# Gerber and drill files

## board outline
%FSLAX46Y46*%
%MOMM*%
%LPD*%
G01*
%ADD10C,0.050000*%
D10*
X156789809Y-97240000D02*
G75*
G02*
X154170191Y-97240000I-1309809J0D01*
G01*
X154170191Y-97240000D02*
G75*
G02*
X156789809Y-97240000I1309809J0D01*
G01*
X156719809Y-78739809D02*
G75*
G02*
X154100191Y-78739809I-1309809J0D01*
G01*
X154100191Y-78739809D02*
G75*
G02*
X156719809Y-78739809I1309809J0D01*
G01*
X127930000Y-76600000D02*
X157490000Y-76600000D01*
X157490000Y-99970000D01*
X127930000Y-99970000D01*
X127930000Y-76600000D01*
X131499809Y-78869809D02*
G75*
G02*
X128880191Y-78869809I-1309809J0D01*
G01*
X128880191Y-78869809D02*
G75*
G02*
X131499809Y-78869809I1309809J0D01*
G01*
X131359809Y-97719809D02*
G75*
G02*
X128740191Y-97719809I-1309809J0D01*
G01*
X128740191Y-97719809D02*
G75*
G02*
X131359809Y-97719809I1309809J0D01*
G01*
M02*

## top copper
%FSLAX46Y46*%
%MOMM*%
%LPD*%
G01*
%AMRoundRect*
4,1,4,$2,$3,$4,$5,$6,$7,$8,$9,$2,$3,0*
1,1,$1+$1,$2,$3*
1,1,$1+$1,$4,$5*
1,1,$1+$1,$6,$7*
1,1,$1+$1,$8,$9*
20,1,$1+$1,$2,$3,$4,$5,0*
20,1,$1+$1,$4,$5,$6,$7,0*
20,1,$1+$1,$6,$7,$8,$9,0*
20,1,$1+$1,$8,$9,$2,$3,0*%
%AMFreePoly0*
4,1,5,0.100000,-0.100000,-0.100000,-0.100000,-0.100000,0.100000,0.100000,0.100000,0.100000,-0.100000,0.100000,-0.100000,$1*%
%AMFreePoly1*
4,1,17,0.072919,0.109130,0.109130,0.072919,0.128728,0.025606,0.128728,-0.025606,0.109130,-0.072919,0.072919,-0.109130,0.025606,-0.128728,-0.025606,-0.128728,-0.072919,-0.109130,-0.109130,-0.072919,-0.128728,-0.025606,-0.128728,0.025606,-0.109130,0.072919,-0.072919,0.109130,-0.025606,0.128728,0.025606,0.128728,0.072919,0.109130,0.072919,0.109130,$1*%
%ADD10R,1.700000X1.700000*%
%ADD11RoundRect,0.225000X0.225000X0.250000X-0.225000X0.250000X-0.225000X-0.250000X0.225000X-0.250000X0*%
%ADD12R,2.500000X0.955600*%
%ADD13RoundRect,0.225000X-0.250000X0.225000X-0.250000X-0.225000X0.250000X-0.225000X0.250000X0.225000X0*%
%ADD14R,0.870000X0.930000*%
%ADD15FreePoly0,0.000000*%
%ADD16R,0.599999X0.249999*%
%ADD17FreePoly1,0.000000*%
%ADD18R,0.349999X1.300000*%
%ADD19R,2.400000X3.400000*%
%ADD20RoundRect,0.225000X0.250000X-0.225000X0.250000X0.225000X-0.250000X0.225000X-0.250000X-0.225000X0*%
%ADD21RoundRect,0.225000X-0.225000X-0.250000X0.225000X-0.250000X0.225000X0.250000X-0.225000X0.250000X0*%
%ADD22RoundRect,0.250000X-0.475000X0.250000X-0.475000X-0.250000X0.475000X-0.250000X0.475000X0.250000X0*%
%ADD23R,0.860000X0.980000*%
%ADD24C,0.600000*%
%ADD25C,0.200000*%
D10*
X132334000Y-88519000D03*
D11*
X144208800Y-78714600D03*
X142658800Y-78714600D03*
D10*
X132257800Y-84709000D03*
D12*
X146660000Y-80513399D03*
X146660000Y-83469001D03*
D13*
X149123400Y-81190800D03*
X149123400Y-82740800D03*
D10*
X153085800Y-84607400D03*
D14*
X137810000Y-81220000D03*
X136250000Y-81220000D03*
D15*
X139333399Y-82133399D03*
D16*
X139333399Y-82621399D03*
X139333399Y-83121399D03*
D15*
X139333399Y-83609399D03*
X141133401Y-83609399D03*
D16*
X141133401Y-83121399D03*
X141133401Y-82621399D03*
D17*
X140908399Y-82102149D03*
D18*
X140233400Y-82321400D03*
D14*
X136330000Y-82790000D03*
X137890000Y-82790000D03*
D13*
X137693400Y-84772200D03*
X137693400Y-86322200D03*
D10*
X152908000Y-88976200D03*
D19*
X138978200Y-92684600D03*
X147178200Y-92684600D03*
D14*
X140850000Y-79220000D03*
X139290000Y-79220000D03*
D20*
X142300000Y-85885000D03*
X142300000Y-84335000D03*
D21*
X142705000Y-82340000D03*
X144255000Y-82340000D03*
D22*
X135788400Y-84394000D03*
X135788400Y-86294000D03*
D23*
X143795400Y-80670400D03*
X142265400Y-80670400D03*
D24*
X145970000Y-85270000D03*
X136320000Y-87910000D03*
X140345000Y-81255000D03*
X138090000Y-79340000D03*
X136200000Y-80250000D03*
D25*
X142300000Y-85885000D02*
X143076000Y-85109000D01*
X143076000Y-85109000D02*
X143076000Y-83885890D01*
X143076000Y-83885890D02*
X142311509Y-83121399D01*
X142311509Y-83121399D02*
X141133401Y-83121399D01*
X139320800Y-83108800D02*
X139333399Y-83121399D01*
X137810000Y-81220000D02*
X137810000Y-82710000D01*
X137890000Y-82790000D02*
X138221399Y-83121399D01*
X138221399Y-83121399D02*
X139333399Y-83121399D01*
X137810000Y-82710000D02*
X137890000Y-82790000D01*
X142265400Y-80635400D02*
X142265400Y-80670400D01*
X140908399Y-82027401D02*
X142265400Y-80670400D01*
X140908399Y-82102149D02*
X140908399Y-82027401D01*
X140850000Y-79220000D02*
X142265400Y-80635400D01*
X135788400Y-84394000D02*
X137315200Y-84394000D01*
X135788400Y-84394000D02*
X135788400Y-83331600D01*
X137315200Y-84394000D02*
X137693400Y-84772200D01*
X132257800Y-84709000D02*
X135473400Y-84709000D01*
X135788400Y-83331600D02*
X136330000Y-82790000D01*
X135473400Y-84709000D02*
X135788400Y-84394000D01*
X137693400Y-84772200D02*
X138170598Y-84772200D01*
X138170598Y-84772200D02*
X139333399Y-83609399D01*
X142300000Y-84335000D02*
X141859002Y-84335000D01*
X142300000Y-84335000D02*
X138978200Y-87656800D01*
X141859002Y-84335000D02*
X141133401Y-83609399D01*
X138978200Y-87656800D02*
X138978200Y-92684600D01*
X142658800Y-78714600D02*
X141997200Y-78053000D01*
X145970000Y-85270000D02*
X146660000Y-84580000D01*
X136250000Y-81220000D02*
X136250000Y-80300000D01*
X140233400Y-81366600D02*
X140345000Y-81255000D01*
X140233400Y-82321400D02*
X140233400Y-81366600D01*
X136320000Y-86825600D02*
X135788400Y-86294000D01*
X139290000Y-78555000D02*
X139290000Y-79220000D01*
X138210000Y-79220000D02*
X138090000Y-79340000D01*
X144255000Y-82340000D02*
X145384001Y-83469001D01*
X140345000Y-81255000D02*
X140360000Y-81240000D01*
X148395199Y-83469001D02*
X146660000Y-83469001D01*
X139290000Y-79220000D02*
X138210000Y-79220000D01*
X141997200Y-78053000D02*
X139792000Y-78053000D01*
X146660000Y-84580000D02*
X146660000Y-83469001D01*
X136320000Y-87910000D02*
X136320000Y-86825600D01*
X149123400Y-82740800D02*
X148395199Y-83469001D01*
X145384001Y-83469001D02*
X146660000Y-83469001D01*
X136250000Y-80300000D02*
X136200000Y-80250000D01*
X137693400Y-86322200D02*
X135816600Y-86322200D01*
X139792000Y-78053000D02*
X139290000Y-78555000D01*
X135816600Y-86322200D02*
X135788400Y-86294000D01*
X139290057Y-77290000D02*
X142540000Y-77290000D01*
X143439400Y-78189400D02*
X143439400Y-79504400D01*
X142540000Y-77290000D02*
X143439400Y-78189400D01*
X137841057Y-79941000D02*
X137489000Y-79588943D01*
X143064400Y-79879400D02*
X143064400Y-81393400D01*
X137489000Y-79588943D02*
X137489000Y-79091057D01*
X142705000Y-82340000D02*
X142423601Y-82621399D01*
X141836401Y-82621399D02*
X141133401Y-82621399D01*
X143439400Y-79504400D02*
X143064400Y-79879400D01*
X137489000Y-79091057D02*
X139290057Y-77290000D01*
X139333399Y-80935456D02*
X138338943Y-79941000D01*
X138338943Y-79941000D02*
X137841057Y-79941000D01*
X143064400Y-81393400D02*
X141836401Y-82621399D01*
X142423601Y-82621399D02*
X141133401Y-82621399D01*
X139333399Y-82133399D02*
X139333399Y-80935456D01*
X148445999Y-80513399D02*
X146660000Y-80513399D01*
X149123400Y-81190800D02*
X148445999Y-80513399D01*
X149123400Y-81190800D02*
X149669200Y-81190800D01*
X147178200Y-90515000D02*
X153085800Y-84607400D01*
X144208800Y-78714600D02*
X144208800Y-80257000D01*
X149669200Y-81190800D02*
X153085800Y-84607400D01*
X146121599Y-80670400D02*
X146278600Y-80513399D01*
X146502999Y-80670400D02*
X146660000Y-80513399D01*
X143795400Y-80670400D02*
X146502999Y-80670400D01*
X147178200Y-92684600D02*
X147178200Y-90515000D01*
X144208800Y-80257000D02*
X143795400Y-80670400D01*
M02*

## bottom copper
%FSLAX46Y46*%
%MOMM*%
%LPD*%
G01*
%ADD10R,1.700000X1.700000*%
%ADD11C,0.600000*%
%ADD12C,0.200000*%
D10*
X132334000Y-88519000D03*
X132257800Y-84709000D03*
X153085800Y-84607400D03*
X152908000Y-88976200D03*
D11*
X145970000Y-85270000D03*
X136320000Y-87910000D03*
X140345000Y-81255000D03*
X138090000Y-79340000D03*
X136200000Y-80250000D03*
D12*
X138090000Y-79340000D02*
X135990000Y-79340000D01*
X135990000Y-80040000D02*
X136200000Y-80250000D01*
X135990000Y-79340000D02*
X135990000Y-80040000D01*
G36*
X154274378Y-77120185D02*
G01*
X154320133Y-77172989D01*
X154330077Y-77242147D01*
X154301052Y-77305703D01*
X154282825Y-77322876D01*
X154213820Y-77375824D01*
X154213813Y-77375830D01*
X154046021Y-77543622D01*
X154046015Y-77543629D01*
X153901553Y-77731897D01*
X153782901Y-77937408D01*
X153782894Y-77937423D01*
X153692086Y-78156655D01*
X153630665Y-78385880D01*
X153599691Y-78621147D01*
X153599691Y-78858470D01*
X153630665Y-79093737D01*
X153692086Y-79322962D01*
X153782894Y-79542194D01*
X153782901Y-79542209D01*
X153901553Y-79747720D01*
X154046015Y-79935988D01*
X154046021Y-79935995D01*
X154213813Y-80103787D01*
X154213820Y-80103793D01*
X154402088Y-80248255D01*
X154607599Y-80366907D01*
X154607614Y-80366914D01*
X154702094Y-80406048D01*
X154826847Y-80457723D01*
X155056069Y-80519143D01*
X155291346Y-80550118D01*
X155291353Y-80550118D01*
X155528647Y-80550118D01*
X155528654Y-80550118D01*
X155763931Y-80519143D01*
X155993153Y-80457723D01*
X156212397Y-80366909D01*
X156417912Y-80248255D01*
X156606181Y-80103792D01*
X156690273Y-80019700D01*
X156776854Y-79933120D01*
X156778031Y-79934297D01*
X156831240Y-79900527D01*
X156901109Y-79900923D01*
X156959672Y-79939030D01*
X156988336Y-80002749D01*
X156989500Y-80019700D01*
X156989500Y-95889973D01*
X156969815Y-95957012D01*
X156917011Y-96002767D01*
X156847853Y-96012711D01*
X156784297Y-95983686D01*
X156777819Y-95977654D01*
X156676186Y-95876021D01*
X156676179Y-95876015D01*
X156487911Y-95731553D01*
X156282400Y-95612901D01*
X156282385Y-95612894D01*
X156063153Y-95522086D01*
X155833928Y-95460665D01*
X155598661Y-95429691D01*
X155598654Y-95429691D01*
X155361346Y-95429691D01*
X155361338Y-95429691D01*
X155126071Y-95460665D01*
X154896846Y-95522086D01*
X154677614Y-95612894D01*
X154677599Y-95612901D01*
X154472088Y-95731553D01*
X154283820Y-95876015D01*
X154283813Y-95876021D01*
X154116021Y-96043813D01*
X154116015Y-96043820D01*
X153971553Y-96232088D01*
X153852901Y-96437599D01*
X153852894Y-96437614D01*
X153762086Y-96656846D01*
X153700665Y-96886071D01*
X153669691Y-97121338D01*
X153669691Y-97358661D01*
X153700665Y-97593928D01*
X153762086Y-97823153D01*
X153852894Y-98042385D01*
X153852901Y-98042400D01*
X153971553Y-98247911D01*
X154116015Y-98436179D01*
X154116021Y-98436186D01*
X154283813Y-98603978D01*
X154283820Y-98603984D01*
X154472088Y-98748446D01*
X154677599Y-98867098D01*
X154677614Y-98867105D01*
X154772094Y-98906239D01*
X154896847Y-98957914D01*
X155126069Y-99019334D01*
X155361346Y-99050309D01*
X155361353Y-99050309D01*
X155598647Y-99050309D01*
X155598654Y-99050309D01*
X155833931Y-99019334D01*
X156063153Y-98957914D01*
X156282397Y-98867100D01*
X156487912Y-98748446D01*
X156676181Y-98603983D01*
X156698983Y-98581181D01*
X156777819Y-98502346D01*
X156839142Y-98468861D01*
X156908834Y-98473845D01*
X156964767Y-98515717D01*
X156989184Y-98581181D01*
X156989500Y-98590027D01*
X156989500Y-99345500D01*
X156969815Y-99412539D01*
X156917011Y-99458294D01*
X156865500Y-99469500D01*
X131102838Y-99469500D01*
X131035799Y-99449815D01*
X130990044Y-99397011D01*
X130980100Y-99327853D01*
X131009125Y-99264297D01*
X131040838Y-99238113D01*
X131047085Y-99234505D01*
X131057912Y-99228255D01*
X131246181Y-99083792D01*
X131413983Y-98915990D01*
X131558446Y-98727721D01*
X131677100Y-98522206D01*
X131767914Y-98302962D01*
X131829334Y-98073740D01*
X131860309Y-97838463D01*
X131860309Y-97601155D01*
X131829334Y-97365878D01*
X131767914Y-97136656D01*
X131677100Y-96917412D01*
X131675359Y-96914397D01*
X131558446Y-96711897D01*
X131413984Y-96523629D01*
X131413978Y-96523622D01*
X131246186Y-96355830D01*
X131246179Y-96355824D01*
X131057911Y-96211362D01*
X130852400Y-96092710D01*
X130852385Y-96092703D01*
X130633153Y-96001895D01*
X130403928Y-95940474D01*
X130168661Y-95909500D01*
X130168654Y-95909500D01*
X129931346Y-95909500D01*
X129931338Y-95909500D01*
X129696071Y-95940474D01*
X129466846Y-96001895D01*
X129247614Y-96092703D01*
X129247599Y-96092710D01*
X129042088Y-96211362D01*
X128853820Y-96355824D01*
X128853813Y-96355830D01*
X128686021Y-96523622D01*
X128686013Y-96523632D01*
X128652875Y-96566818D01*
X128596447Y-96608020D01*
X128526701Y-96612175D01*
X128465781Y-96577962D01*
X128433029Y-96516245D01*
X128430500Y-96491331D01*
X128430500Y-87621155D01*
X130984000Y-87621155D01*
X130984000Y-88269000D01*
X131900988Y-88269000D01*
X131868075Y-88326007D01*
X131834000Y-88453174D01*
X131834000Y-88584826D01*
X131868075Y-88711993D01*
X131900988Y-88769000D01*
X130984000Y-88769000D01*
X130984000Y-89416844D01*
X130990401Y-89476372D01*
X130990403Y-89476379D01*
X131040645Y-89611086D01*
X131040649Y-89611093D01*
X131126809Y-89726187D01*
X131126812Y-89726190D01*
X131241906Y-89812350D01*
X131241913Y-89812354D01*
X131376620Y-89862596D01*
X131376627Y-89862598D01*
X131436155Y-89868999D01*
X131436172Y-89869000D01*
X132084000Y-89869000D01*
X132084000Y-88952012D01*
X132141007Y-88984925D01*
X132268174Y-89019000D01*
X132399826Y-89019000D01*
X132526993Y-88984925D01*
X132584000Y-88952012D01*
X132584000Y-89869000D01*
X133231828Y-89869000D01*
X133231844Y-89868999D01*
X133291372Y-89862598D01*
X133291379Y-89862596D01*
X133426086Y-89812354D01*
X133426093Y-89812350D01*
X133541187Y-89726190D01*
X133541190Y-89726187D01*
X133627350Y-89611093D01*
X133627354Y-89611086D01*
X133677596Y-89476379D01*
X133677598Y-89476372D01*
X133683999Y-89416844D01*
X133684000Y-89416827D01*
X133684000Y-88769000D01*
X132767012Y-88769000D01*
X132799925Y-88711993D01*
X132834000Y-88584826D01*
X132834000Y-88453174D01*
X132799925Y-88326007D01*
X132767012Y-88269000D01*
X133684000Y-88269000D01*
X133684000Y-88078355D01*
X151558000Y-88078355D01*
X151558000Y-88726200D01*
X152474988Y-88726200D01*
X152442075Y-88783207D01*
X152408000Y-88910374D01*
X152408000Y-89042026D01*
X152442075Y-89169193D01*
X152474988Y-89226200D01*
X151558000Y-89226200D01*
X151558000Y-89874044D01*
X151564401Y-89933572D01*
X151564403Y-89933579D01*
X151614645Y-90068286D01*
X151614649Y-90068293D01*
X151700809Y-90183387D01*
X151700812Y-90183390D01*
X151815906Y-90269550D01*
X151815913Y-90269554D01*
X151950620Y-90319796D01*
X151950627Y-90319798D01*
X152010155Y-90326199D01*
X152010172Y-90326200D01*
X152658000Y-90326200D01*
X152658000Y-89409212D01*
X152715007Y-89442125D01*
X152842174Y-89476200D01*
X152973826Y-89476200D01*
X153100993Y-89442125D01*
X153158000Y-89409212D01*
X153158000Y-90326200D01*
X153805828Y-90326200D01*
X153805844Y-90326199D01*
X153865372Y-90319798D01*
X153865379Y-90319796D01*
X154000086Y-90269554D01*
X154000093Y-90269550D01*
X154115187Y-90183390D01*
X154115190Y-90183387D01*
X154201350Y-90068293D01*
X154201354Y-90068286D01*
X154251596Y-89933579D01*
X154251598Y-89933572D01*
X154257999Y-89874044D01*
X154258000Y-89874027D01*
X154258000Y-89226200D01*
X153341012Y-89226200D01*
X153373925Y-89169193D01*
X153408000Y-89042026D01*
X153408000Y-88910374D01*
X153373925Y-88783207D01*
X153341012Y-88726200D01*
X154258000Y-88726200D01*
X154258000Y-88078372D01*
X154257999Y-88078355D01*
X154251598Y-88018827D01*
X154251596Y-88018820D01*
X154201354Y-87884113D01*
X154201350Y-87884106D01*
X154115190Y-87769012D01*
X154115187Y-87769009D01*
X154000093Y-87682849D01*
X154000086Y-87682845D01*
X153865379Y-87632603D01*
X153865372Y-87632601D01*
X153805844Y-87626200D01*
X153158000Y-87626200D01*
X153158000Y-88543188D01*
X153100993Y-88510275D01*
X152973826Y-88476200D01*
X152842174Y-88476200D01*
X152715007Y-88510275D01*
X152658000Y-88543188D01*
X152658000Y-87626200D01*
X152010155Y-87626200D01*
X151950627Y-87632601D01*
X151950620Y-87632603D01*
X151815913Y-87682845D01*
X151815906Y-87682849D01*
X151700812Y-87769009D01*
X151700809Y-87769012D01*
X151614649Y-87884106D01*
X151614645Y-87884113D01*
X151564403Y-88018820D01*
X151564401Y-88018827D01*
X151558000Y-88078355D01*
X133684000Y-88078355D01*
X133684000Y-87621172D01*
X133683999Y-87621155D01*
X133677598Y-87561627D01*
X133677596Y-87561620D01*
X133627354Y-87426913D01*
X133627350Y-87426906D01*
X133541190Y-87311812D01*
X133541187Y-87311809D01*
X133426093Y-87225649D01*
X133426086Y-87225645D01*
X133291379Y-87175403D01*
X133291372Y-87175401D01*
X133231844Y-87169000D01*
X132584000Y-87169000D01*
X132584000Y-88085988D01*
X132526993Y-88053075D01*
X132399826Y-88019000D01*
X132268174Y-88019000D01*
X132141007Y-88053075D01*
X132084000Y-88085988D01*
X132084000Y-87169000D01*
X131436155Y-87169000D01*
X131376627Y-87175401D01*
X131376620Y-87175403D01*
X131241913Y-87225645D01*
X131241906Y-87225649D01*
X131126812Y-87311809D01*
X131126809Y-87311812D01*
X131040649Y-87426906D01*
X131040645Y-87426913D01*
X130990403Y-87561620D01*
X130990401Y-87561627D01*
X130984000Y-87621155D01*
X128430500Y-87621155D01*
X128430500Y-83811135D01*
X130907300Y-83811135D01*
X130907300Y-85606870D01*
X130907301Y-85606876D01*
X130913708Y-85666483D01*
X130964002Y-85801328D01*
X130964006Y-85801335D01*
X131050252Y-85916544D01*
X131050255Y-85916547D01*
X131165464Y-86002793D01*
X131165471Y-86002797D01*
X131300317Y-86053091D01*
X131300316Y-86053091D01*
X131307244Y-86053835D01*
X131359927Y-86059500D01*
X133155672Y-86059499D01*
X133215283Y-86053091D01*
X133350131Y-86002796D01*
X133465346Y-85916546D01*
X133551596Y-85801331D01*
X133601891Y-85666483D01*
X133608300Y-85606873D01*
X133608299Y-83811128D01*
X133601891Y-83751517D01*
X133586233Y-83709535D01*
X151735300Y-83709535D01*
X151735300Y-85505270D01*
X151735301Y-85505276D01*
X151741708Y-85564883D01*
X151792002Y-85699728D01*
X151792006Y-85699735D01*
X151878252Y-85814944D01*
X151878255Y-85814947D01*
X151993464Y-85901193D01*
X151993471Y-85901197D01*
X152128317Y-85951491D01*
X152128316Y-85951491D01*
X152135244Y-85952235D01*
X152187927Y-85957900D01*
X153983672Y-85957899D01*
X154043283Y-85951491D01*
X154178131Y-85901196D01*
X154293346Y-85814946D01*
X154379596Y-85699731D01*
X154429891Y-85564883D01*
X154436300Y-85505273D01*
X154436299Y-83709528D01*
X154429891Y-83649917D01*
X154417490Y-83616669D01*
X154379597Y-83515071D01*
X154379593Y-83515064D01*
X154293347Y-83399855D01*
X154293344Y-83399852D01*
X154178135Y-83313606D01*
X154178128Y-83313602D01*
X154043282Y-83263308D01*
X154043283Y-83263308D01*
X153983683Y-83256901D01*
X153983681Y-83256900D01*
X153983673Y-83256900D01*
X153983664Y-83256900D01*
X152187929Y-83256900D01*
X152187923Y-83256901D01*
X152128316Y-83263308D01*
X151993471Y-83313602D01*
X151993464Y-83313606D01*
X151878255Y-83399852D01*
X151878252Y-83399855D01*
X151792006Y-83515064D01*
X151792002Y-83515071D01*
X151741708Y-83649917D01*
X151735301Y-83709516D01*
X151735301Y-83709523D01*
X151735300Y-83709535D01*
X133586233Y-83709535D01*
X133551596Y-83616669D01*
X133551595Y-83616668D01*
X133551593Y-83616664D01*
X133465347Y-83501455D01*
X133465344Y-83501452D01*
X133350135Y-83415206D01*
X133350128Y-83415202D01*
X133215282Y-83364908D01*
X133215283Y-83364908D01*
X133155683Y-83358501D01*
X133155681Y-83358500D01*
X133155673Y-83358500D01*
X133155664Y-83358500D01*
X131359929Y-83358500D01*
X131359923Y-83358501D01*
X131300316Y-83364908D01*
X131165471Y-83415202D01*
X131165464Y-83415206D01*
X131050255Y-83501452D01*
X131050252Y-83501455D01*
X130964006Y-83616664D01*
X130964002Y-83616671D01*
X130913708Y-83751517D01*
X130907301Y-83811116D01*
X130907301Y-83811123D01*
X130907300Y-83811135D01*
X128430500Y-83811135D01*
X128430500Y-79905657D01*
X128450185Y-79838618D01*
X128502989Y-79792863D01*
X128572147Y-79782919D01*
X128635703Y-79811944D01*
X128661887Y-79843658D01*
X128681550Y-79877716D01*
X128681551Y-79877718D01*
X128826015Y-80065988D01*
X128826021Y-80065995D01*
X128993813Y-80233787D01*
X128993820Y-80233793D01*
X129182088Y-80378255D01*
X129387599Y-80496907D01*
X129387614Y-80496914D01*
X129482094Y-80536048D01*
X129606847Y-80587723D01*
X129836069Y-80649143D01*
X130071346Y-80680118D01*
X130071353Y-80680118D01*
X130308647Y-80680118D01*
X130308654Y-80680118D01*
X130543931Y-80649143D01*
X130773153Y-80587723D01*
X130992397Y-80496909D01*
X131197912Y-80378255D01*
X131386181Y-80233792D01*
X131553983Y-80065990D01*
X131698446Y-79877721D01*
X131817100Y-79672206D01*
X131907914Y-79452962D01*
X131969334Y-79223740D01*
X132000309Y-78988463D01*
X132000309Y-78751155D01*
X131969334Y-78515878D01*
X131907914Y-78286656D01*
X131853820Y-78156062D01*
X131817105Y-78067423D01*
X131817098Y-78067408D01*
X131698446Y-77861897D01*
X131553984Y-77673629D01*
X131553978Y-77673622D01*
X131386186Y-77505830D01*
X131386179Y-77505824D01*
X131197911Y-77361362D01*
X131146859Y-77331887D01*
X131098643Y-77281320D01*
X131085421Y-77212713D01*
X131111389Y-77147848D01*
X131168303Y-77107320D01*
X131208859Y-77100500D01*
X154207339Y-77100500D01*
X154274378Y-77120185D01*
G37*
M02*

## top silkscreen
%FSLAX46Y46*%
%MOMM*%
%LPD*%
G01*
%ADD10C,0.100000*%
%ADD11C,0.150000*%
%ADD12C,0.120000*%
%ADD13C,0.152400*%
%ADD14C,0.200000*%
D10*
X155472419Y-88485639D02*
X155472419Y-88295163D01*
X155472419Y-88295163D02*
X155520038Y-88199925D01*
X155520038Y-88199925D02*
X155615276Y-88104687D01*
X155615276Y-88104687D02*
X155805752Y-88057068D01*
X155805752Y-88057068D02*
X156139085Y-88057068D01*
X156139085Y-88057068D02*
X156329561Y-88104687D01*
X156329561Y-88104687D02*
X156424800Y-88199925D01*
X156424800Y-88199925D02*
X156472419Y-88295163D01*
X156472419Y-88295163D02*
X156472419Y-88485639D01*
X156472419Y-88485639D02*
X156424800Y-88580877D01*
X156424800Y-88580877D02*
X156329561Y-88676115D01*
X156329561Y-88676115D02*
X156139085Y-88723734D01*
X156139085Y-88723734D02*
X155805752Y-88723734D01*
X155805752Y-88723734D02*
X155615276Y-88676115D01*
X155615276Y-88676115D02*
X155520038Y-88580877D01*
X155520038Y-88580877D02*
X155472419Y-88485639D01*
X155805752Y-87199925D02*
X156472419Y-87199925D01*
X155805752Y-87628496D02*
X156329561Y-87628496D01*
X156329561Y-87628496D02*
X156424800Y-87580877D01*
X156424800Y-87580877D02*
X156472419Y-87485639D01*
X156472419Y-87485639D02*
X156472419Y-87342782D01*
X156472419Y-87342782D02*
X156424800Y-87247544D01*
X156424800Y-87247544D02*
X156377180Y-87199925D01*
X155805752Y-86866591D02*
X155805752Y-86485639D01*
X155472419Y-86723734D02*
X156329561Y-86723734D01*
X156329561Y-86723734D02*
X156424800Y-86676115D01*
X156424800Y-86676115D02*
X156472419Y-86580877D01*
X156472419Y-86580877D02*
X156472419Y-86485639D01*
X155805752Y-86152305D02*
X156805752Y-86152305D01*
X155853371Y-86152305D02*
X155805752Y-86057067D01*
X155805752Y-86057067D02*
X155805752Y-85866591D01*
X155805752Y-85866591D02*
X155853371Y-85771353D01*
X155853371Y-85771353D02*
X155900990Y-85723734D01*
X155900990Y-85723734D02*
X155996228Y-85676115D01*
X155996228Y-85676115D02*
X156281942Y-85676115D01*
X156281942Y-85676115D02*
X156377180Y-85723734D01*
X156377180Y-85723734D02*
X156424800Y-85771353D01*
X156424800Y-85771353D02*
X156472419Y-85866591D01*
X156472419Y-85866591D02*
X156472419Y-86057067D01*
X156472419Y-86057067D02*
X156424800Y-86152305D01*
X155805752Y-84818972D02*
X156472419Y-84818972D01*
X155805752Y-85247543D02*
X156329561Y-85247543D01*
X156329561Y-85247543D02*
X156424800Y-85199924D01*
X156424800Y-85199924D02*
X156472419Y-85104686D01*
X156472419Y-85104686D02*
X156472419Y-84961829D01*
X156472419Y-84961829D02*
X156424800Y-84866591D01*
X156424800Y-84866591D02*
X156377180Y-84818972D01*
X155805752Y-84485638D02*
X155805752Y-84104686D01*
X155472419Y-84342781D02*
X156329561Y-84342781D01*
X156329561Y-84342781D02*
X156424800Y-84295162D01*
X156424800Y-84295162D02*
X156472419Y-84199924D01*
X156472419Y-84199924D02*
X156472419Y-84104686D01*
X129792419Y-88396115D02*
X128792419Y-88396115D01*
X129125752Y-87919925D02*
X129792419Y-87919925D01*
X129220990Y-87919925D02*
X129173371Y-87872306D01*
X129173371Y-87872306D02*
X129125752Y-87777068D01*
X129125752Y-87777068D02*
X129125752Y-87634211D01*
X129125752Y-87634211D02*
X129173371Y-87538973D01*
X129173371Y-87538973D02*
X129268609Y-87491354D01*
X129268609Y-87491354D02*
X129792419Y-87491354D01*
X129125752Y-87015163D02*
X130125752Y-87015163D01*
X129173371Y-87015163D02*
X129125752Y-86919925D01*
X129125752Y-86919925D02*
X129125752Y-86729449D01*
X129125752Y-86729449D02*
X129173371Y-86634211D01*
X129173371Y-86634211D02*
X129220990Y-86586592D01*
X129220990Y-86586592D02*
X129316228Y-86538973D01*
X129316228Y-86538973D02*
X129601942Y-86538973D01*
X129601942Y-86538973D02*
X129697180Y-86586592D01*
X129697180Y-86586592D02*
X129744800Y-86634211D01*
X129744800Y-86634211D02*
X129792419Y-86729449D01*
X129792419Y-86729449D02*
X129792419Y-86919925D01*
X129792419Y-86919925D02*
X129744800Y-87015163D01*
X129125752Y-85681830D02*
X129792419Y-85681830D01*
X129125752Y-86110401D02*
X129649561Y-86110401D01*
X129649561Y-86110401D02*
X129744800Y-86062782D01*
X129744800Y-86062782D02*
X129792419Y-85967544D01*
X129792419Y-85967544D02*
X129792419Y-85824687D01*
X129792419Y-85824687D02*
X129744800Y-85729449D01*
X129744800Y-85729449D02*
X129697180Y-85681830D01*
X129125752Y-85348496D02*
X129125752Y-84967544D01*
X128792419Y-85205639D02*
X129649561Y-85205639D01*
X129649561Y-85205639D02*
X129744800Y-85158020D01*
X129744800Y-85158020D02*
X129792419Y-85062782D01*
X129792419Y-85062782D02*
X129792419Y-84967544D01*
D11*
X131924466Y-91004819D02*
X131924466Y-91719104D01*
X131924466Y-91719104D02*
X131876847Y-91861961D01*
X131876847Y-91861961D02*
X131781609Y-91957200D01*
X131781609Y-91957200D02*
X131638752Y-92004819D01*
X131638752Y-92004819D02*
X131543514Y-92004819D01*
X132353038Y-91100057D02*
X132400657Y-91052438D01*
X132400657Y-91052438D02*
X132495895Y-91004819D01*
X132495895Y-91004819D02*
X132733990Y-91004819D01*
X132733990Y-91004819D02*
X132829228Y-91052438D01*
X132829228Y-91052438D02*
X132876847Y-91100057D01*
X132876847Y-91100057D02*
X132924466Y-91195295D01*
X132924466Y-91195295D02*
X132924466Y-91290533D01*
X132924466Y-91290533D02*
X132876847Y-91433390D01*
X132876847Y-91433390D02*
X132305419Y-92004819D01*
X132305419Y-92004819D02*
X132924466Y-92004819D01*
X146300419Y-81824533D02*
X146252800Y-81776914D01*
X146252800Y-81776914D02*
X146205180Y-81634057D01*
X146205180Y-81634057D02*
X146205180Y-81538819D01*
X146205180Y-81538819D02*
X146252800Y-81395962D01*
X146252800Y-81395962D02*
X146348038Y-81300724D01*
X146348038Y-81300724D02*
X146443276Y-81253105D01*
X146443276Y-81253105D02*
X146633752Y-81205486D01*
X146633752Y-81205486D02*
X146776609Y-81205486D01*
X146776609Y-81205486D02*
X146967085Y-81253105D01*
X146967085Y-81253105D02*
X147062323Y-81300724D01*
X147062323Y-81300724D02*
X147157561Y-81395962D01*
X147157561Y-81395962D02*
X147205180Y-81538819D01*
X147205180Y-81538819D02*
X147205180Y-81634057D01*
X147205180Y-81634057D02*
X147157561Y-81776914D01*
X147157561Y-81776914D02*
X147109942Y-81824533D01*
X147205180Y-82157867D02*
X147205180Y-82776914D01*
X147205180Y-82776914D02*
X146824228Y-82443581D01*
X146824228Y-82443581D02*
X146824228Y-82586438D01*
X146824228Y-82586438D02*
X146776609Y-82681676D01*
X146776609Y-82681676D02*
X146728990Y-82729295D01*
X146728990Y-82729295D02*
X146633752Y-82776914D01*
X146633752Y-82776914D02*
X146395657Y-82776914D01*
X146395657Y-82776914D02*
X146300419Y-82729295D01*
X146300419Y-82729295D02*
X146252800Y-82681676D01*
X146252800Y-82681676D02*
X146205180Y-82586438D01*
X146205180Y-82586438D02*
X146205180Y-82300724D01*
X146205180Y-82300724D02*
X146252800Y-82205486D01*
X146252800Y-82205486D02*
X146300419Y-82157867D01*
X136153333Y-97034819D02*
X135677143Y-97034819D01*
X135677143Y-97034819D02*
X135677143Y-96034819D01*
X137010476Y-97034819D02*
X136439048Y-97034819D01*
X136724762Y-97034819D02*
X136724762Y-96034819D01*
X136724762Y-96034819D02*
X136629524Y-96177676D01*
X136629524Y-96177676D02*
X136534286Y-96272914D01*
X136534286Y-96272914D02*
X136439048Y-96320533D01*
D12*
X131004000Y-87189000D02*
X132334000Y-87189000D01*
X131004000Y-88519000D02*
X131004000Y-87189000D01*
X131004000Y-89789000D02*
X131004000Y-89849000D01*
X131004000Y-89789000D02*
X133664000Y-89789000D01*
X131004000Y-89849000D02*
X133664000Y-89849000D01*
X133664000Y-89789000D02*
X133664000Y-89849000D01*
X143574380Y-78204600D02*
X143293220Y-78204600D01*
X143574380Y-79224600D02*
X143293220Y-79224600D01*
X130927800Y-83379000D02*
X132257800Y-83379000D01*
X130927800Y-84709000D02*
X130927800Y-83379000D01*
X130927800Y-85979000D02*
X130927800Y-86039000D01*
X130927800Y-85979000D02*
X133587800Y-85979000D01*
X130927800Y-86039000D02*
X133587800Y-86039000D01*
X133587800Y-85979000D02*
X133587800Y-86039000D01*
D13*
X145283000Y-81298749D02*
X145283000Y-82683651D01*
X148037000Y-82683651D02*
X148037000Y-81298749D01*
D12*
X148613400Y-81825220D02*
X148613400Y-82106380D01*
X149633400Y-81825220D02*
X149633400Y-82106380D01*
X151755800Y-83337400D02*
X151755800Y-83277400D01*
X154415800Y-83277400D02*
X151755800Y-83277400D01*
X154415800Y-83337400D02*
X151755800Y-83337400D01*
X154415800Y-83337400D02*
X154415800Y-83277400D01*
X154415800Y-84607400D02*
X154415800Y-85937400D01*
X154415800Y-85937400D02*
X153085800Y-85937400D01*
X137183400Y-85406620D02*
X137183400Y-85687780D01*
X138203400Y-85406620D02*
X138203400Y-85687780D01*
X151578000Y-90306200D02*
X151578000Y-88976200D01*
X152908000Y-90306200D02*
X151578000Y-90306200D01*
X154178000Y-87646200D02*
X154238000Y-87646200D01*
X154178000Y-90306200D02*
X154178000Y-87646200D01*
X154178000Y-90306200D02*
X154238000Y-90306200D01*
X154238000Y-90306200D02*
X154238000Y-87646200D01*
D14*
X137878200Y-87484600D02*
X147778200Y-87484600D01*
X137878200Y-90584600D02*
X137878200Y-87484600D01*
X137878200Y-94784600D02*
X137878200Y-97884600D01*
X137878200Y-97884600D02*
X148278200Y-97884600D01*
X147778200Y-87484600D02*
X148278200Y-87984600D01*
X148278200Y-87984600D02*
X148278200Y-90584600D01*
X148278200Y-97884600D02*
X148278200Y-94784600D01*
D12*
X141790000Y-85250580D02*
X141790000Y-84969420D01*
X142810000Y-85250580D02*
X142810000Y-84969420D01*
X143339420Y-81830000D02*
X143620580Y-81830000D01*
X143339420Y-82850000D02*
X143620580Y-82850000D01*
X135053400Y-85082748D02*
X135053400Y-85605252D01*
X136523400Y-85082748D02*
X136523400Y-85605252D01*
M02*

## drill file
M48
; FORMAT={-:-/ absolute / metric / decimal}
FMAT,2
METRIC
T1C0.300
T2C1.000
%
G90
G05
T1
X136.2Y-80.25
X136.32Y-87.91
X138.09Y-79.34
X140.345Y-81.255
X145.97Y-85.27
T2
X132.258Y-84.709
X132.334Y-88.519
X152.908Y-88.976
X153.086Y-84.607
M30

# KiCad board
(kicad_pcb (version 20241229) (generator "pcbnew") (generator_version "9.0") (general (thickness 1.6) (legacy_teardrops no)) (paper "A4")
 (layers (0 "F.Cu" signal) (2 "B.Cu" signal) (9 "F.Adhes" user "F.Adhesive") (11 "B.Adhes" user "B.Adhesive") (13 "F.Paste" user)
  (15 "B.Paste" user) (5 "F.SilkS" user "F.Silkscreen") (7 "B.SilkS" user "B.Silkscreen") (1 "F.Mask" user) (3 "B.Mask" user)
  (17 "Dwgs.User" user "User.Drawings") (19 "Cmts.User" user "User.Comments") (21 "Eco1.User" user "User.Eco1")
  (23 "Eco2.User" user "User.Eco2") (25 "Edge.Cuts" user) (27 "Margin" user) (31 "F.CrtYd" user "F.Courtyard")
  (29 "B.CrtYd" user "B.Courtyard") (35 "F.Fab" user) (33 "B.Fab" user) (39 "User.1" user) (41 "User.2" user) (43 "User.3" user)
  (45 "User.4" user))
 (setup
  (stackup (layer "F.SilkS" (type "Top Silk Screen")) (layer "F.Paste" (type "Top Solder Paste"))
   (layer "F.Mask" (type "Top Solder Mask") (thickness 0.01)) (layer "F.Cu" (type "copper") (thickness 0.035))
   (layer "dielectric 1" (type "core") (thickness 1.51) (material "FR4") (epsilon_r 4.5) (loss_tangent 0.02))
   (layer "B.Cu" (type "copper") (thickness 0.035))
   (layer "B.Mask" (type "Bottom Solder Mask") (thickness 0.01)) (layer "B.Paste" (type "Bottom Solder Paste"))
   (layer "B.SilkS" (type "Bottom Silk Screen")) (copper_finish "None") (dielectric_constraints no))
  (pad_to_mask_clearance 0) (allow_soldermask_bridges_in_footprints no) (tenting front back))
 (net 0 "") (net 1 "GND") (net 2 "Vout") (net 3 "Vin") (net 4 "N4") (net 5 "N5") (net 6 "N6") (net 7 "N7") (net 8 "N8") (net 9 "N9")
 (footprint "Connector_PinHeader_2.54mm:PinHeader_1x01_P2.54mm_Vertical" (layer "F.Cu") (at 132.334 88.519)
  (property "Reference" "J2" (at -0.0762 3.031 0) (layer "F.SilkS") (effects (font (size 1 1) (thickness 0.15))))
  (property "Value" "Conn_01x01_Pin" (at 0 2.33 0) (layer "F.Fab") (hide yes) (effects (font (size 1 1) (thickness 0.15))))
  (fp_line (start -1.33 -1.33) (end 0 -1.33) (stroke (width 0.12) (type solid)) (layer "F.SilkS"))
  (fp_line (start -1.33 0) (end -1.33 -1.33) (stroke (width 0.12) (type solid)) (layer "F.SilkS"))
  (fp_line (start -1.33 1.27) (end -1.33 1.33) (stroke (width 0.12) (type solid)) (layer "F.SilkS"))
  (fp_line (start -1.33 1.27) (end 1.33 1.27) (stroke (width 0.12) (type solid)) (layer "F.SilkS"))
  (fp_line (start -1.33 1.33) (end 1.33 1.33) (stroke (width 0.12) (type solid)) (layer "F.SilkS"))
  (fp_line (start 1.33 1.27) (end 1.33 1.33) (stroke (width 0.12) (type solid)) (layer "F.SilkS"))
  (pad "1" thru_hole rect (at 0 0) (size 1.7 1.7) (drill 1) (layers "*.Cu" "*.Mask") (remove_unused_layers no) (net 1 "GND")))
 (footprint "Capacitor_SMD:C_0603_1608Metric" (layer "F.Cu") (at 143.4338 78.7146 180)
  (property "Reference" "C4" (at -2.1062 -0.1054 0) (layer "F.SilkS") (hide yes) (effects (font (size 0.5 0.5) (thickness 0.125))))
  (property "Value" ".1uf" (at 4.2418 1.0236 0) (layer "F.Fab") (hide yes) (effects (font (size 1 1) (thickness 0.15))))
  (fp_line (start -0.14058 0.51) (end 0.14058 0.51) (stroke (width 0.12) (type solid)) (layer "F.SilkS"))
  (fp_line (start -0.14058 -0.51) (end 0.14058 -0.51) (stroke (width 0.12) (type solid)) (layer "F.SilkS"))
  (pad "1" smd roundrect (at -0.775 0 180) (size 0.9 0.95) (layers "F.Cu" "F.Mask" "F.Paste") (roundrect_rratio 0.25) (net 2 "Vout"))
  (pad "2" smd roundrect (at 0.775 0 180) (size 0.9 0.95) (layers "F.Cu" "F.Mask" "F.Paste") (roundrect_rratio 0.25) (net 1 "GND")))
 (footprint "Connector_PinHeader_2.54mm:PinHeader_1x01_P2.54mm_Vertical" (layer "F.Cu") (at 132.2578 84.709)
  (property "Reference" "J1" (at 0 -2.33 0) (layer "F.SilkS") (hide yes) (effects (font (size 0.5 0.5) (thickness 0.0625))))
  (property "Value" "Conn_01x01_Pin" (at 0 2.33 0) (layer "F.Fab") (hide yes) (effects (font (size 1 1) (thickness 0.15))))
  (fp_line (start -1.33 -1.33) (end 0 -1.33) (stroke (width 0.12) (type solid)) (layer "F.SilkS"))
  (fp_line (start -1.33 0) (end -1.33 -1.33) (stroke (width 0.12) (type solid)) (layer "F.SilkS"))
  (fp_line (start -1.33 1.27) (end -1.33 1.33) (stroke (width 0.12) (type solid)) (layer "F.SilkS"))
  (fp_line (start -1.33 1.27) (end 1.33 1.27) (stroke (width 0.12) (type solid)) (layer "F.SilkS"))
  (fp_line (start -1.33 1.33) (end 1.33 1.33) (stroke (width 0.12) (type solid)) (layer "F.SilkS"))
  (fp_line (start 1.33 1.27) (end 1.33 1.33) (stroke (width 0.12) (type solid)) (layer "F.SilkS"))
  (pad "1" thru_hole rect (at 0 0) (size 1.7 1.7) (drill 1) (layers "*.Cu" "*.Mask") (remove_unused_layers no) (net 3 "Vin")))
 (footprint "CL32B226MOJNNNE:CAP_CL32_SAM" (layer "F.Cu") (at 146.66 81.9912 -90)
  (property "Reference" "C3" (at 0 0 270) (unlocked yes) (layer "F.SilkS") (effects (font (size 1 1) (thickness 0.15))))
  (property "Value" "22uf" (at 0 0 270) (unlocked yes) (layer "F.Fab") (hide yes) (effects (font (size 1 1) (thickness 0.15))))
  (fp_line (start -0.692451 1.377) (end 0.692451 1.377) (stroke (width 0.1524) (type solid)) (layer "F.SilkS"))
  (fp_line (start 0.692451 -1.377) (end -0.692451 -1.377) (stroke (width 0.1524) (type solid)) (layer "F.SilkS"))
  (pad "1" smd rect (at -1.477801 0 270) (size 0.9556 2.5) (layers "F.Cu" "F.Mask" "F.Paste") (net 2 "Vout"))
  (pad "2" smd rect (at 1.477801 0 270) (size 0.9556 2.5) (layers "F.Cu" "F.Mask" "F.Paste") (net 1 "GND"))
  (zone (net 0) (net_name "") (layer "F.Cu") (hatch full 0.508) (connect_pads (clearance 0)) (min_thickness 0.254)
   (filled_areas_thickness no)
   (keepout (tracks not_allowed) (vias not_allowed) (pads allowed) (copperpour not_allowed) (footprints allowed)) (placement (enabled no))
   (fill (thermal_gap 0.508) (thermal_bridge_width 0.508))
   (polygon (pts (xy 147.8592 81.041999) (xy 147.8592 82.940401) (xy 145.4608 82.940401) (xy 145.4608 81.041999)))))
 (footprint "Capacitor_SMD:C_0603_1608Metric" (layer "F.Cu") (at 149.1234 81.9658 -90)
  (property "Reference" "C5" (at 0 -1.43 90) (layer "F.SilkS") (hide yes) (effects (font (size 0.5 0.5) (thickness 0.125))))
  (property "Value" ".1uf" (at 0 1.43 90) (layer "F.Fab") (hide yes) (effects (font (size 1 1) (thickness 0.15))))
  (fp_line (start -0.14058 0.51) (end 0.14058 0.51) (stroke (width 0.12) (type solid)) (layer "F.SilkS"))
  (fp_line (start -0.14058 -0.51) (end 0.14058 -0.51) (stroke (width 0.12) (type solid)) (layer "F.SilkS"))
  (pad "1" smd roundrect (at -0.775 0 270) (size 0.9 0.95) (layers "F.Cu" "F.Mask" "F.Paste") (roundrect_rratio 0.25) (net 2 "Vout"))
  (pad "2" smd roundrect (at 0.775 0 270) (size 0.9 0.95) (layers "F.Cu" "F.Mask" "F.Paste") (roundrect_rratio 0.25) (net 1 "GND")))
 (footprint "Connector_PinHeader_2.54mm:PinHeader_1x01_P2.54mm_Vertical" (layer "F.Cu") (at 153.0858 84.6074 180)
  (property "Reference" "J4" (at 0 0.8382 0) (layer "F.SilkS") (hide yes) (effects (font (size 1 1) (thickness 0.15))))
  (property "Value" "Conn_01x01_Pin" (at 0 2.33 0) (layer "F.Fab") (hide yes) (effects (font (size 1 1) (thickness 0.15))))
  (fp_line (start 1.33 1.27) (end 1.33 1.33) (stroke (width 0.12) (type solid)) (layer "F.SilkS"))
  (fp_line (start -1.33 1.33) (end 1.33 1.33) (stroke (width 0.12) (type solid)) (layer "F.SilkS"))
  (fp_line (start -1.33 1.27) (end 1.33 1.27) (stroke (width 0.12) (type solid)) (layer "F.SilkS"))
  (fp_line (start -1.33 1.27) (end -1.33 1.33) (stroke (width 0.12) (type solid)) (layer "F.SilkS"))
  (fp_line (start -1.33 0) (end -1.33 -1.33) (stroke (width 0.12) (type solid)) (layer "F.SilkS"))
  (fp_line (start -1.33 -1.33) (end 0 -1.33) (stroke (width 0.12) (type solid)) (layer "F.SilkS"))
  (pad "1" thru_hole rect (at 0 0 180) (size 1.7 1.7) (drill 1) (layers "*.Cu" "*.Mask") (remove_unused_layers no) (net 2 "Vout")))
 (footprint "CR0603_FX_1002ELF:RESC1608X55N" (layer "F.Cu") (at 137.03 81.22 180)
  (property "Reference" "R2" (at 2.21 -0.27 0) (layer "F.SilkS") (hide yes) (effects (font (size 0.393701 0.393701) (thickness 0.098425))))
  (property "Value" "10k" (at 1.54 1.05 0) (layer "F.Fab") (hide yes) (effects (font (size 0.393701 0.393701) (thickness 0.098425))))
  (pad "1" smd rect (at -0.78 0 180) (size 0.87 0.93) (layers "F.Cu" "F.Mask" "F.Paste") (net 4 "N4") (solder_mask_margin 0.102))
  (pad "2" smd rect (at 0.78 0 180) (size 0.87 0.93) (layers "F.Cu" "F.Mask" "F.Paste") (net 1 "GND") (solder_mask_margin 0.102)))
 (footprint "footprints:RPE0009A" (layer "F.Cu") (at 140.2334 82.871399)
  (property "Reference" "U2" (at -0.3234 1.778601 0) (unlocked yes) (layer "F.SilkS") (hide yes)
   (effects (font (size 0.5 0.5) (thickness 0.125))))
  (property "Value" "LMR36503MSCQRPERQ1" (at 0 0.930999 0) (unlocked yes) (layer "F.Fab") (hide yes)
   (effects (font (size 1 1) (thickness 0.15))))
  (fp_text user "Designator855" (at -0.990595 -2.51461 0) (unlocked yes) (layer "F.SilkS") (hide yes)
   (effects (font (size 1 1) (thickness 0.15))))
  (pad "1" smd custom (at -0.900001 -0.738) (size 0.2 0.2) (layers "F.Cu" "F.Mask" "F.Paste") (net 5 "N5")
   (options (clearance outline) (anchor rect)) (primitives))
  (pad "2" smd rect (at -0.900001 -0.25) (size 0.599999 0.249999) (layers "F.Cu" "F.Mask" "F.Paste") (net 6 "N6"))
  (pad "3" smd rect (at -0.900001 0.25) (size 0.599999 0.249999) (layers "F.Cu" "F.Mask" "F.Paste") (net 4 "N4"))
  (pad "4" smd custom (at -0.900001 0.738) (size 0.2 0.2) (layers "F.Cu" "F.Mask" "F.Paste") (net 3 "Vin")
   (options (clearance outline) (anchor rect)) (primitives))
  (pad "5" smd custom (at 0.900001 0.738) (size 0.2 0.2) (layers "F.Cu" "F.Mask" "F.Paste") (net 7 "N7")
   (options (clearance outline) (anchor rect)) (primitives))
  (pad "6" smd rect (at 0.900001 0.25) (size 0.599999 0.249999) (layers "F.Cu" "F.Mask" "F.Paste") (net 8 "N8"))
  (pad "7" smd rect (at 0.900001 -0.25) (size 0.599999 0.249999) (layers "F.Cu" "F.Mask" "F.Paste") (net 5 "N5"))
  (pad "8" smd custom (at 0.674999 -0.76925) (size 0.262501 0.262501) (layers "F.Cu" "F.Mask" "F.Paste") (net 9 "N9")
   (thermal_bridge_angle 90) (options (clearance outline) (anchor circle)) (primitives))
  (pad "9" smd rect (at 0 -0.549999) (size 0.349999 1.3) (layers "F.Cu" "F.Mask") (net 1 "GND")))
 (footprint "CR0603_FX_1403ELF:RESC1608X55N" (layer "F.Cu") (at 137.11 82.79)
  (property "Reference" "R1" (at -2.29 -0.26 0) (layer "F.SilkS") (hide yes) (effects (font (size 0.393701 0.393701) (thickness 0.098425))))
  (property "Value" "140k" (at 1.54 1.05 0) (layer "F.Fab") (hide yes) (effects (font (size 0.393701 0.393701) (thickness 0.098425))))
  (pad "1" smd rect (at -0.78 0) (size 0.87 0.93) (layers "F.Cu" "F.Mask" "F.Paste") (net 3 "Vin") (solder_mask_margin 0.102))
  (pad "2" smd rect (at 0.78 0) (size 0.87 0.93) (layers "F.Cu" "F.Mask" "F.Paste") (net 4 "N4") (solder_mask_margin 0.102)))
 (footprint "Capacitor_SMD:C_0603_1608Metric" (layer "F.Cu") (at 137.6934 85.5472 -90)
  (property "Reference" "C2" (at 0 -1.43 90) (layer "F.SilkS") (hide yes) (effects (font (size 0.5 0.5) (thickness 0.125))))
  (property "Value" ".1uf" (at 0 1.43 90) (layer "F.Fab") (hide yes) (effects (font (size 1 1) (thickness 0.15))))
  (fp_line (start -0.14058 0.51) (end 0.14058 0.51) (stroke (width 0.12) (type solid)) (layer "F.SilkS"))
  (fp_line (start -0.14058 -0.51) (end 0.14058 -0.51) (stroke (width 0.12) (type solid)) (layer "F.SilkS"))
  (pad "1" smd roundrect (at -0.775 0 270) (size 0.9 0.95) (layers "F.Cu" "F.Mask" "F.Paste") (roundrect_rratio 0.25) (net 3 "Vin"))
  (pad "2" smd roundrect (at 0.775 0 270) (size 0.9 0.95) (layers "F.Cu" "F.Mask" "F.Paste") (roundrect_rratio 0.25) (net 1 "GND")))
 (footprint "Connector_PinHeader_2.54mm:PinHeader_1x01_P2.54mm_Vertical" (layer "F.Cu") (at 152.908 88.9762 90)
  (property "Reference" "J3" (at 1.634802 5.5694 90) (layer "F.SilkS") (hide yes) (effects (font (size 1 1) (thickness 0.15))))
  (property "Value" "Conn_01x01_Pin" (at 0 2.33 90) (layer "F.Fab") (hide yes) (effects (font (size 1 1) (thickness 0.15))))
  (fp_line (start -1.33 -1.33) (end 0 -1.33) (stroke (width 0.12) (type solid)) (layer "F.SilkS"))
  (fp_line (start -1.33 0) (end -1.33 -1.33) (stroke (width 0.12) (type solid)) (layer "F.SilkS"))
  (fp_line (start 1.33 1.27) (end 1.33 1.33) (stroke (width 0.12) (type solid)) (layer "F.SilkS"))
  (fp_line (start -1.33 1.27) (end 1.33 1.27) (stroke (width 0.12) (type solid)) (layer "F.SilkS"))
  (fp_line (start -1.33 1.27) (end -1.33 1.33) (stroke (width 0.12) (type solid)) (layer "F.SilkS"))
  (fp_line (start -1.33 1.33) (end 1.33 1.33) (stroke (width 0.12) (type solid)) (layer "F.SilkS"))
  (pad "1" thru_hole rect (at 0 0 90) (size 1.7 1.7) (drill 1) (layers "*.Cu" "*.Mask") (remove_unused_layers no) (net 1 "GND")))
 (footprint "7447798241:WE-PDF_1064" (layer "F.Cu") (at 143.0782 92.6846)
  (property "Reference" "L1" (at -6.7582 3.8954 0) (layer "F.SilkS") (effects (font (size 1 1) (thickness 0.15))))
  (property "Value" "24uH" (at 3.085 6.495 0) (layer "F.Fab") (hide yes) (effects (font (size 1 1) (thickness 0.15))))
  (fp_line (start -5.2 -5.2) (end 4.7 -5.2) (stroke (width 0.2) (type solid)) (layer "F.SilkS"))
  (fp_line (start -5.2 -2.1) (end -5.2 -5.2) (stroke (width 0.2) (type solid)) (layer "F.SilkS"))
  (fp_line (start -5.2 2.1) (end -5.2 5.2) (stroke (width 0.2) (type solid)) (layer "F.SilkS"))
  (fp_line (start -5.2 5.2) (end 5.2 5.2) (stroke (width 0.2) (type solid)) (layer "F.SilkS"))
  (fp_line (start 4.7 -5.2) (end 5.2 -4.7) (stroke (width 0.2) (type solid)) (layer "F.SilkS"))
  (fp_line (start 5.2 -4.7) (end 5.2 -2.1) (stroke (width 0.2) (type solid)) (layer "F.SilkS"))
  (fp_line (start 5.2 5.2) (end 5.2 2.1) (stroke (width 0.2) (type solid)) (layer "F.SilkS"))
  (pad "1" smd rect (at -4.1 0) (size 2.4 3.4) (layers "F.Cu" "F.Mask" "F.Paste") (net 7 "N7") (solder_mask_margin 0.102))
  (pad "2" smd rect (at 4.1 0) (size 2.4 3.4) (layers "F.Cu" "F.Mask" "F.Paste") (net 2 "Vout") (solder_mask_margin 0.102)))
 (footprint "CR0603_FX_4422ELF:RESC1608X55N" (layer "F.Cu") (at 140.07 79.22 180)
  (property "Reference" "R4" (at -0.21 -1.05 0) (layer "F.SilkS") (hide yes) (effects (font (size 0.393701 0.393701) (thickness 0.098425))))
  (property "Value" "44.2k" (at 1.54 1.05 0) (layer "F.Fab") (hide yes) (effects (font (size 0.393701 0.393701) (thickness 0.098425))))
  (pad "1" smd rect (at -0.78 0 180) (size 0.87 0.93) (layers "F.Cu" "F.Mask" "F.Paste") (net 9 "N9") (solder_mask_margin 0.102))
  (pad "2" smd rect (at 0.78 0 180) (size 0.87 0.93) (layers "F.Cu" "F.Mask" "F.Paste") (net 1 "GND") (solder_mask_margin 0.102)))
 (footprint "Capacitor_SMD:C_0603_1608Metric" (layer "F.Cu") (at 142.3 85.11 90)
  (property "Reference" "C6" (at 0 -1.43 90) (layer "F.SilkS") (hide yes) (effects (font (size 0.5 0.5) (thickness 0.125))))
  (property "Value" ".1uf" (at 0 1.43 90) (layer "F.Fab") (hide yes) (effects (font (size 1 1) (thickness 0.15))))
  (fp_line (start -0.14058 -0.51) (end 0.14058 -0.51) (stroke (width 0.12) (type solid)) (layer "F.SilkS"))
  (fp_line (start -0.14058 0.51) (end 0.14058 0.51) (stroke (width 0.12) (type solid)) (layer "F.SilkS"))
  (pad "1" smd roundrect (at -0.775 0 90) (size 0.9 0.95) (layers "F.Cu" "F.Mask" "F.Paste") (roundrect_rratio 0.25) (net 8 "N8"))
  (pad "2" smd roundrect (at 0.775 0 90) (size 0.9 0.95) (layers "F.Cu" "F.Mask" "F.Paste") (roundrect_rratio 0.25) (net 7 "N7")))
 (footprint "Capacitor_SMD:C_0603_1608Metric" (layer "F.Cu") (at 143.48 82.34)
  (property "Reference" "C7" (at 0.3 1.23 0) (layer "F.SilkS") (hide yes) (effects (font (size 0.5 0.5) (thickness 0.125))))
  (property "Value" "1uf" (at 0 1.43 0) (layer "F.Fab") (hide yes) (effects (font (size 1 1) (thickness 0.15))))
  (fp_line (start -0.14058 -0.51) (end 0.14058 -0.51) (stroke (width 0.12) (type solid)) (layer "F.SilkS"))
  (fp_line (start -0.14058 0.51) (end 0.14058 0.51) (stroke (width 0.12) (type solid)) (layer "F.SilkS"))
  (pad "1" smd roundrect (at -0.775 0) (size 0.9 0.95) (layers "F.Cu" "F.Mask" "F.Paste") (roundrect_rratio 0.25) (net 5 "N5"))
  (pad "2" smd roundrect (at 0.775 0) (size 0.9 0.95) (layers "F.Cu" "F.Mask" "F.Paste") (roundrect_rratio 0.25) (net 1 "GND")))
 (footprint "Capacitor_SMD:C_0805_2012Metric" (layer "F.Cu") (at 135.7884 85.344 -90)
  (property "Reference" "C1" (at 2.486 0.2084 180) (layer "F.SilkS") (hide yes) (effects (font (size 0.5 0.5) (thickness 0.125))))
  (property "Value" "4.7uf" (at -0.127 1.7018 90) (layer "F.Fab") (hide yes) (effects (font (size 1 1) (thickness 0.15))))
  (fp_line (start -0.261252 0.735) (end 0.261252 0.735) (stroke (width 0.12) (type solid)) (layer "F.SilkS"))
  (fp_line (start -0.261252 -0.735) (end 0.261252 -0.735) (stroke (width 0.12) (type solid)) (layer "F.SilkS"))
  (pad "1" smd roundrect (at -0.95 0 270) (size 1 1.45) (layers "F.Cu" "F.Mask" "F.Paste") (roundrect_rratio 0.25) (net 3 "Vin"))
  (pad "2" smd roundrect (at 0.95 0 270) (size 1 1.45) (layers "F.Cu" "F.Mask" "F.Paste") (roundrect_rratio 0.25) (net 1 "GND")))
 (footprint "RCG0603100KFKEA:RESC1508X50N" (layer "F.Cu") (at 143.0304 80.6704 180)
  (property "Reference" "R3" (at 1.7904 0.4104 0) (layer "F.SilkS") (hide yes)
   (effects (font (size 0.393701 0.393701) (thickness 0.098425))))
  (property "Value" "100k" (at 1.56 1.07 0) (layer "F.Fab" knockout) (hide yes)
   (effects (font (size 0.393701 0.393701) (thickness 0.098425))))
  (pad "1" smd rect (at -0.765 0 180) (size 0.86 0.98) (layers "F.Cu" "F.Mask" "F.Paste") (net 2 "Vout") (solder_mask_margin 0.102))
  (pad "2" smd rect (at 0.765 0 180) (size 0.86 0.98) (layers "F.Cu" "F.Mask" "F.Paste") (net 9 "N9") (solder_mask_margin 0.102)))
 (gr_circle (center 155.48 97.24) (end 155.32 95.94) (stroke (width 0.05) (type default)) (fill no) (layer "Edge.Cuts"))
 (gr_circle (center 155.41 78.739809) (end 155.25 77.439809) (stroke (width 0.05) (type default)) (fill no) (layer "Edge.Cuts"))
 (gr_rect (start 127.93 76.6) (end 157.49 99.97) (stroke (width 0.05) (type default)) (fill no) (layer "Edge.Cuts"))
 (gr_circle (center 130.19 78.869809) (end 130.03 77.569809) (stroke (width 0.05) (type default)) (fill no) (layer "Edge.Cuts"))
 (gr_circle (center 130.05 97.719809) (end 129.89 96.419809) (stroke (width 0.05) (type default)) (fill no) (layer "Edge.Cuts"))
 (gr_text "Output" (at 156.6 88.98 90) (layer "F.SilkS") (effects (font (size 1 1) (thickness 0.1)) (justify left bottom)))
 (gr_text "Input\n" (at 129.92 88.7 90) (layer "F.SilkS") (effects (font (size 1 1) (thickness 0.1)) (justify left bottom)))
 (segment (start 142.3 85.885) (end 143.076 85.109) (width 0.2) (layer "F.Cu") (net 8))
 (segment (start 143.076 85.109) (end 143.076 83.88589) (width 0.2) (layer "F.Cu") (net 8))
 (segment (start 143.076 83.88589) (end 142.311509 83.121399) (width 0.2) (layer "F.Cu") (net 8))
 (segment (start 142.311509 83.121399) (end 141.133401 83.121399) (width 0.2) (layer "F.Cu") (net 8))
 (segment (start 139.3208 83.1088) (end 139.333399 83.121399) (width 0.2) (layer "F.Cu") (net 4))
 (segment (start 137.81 81.22) (end 137.81 82.71) (width 0.2) (layer "F.Cu") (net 4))
 (segment (start 137.89 82.79) (end 138.221399 83.121399) (width 0.2) (layer "F.Cu") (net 4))
 (segment (start 138.221399 83.121399) (end 139.333399 83.121399) (width 0.2) (layer "F.Cu") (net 4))
 (segment (start 137.81 82.71) (end 137.89 82.79) (width 0.2) (layer "F.Cu") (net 4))
 (segment (start 142.2654 80.6354) (end 142.2654 80.6704) (width 0.2) (layer "F.Cu") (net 9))
 (segment (start 140.908399 82.027401) (end 142.2654 80.6704) (width 0.2) (layer "F.Cu") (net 9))
 (segment (start 140.908399 82.102149) (end 140.908399 82.027401) (width 0.2) (layer "F.Cu") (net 9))
 (segment (start 140.85 79.22) (end 142.2654 80.6354) (width 0.2) (layer "F.Cu") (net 9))
 (segment (start 135.7884 84.394) (end 137.3152 84.394) (width 0.2) (layer "F.Cu") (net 3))
 (segment (start 135.7884 84.394) (end 135.7884 83.3316) (width 0.2) (layer "F.Cu") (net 3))
 (segment (start 137.3152 84.394) (end 137.6934 84.7722) (width 0.2) (layer "F.Cu") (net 3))
 (segment (start 132.2578 84.709) (end 135.4734 84.709) (width 0.2) (layer "F.Cu") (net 3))
 (segment (start 135.7884 83.3316) (end 136.33 82.79) (width 0.2) (layer "F.Cu") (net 3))
 (segment (start 135.4734 84.709) (end 135.7884 84.394) (width 0.2) (layer "F.Cu") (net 3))
 (segment (start 137.6934 84.7722) (end 138.170598 84.7722) (width 0.2) (layer "F.Cu") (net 3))
 (segment (start 138.170598 84.7722) (end 139.333399 83.609399) (width 0.2) (layer "F.Cu") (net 3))
 (segment (start 142.3 84.335) (end 141.859002 84.335) (width 0.2) (layer "F.Cu") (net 7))
 (segment (start 142.3 84.335) (end 138.9782 87.6568) (width 0.2) (layer "F.Cu") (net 7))
 (segment (start 141.859002 84.335) (end 141.133401 83.609399) (width 0.2) (layer "F.Cu") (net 7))
 (segment (start 138.9782 87.6568) (end 138.9782 92.6846) (width 0.2) (layer "F.Cu") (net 7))
 (segment (start 142.6588 78.7146) (end 141.9972 78.053) (width 0.2) (layer "F.Cu") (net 1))
 (segment (start 145.97 85.27) (end 146.66 84.58) (width 0.2) (layer "F.Cu") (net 1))
 (segment (start 136.25 81.22) (end 136.25 80.3) (width 0.2) (layer "F.Cu") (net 1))
 (segment (start 140.2334 81.3666) (end 140.345 81.255) (width 0.2) (layer "F.Cu") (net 1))
 (segment (start 140.2334 82.3214) (end 140.2334 81.3666) (width 0.2) (layer "F.Cu") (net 1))
 (segment (start 136.32 86.8256) (end 135.7884 86.294) (width 0.2) (layer "F.Cu") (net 1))
 (segment (start 139.29 78.555) (end 139.29 79.22) (width 0.2) (layer "F.Cu") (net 1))
 (segment (start 138.21 79.22) (end 138.09 79.34) (width 0.2) (layer "F.Cu") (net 1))
 (segment (start 144.255 82.34) (end 145.384001 83.469001) (width 0.2) (layer "F.Cu") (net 1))
 (segment (start 140.345 81.255) (end 140.36 81.24) (width 0.2) (layer "F.Cu") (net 1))
 (segment (start 148.395199 83.469001) (end 146.66 83.469001) (width 0.2) (layer "F.Cu") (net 1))
 (segment (start 139.29 79.22) (end 138.21 79.22) (width 0.2) (layer "F.Cu") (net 1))
 (segment (start 141.9972 78.053) (end 139.792 78.053) (width 0.2) (layer "F.Cu") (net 1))
 (segment (start 146.66 84.58) (end 146.66 83.469001) (width 0.2) (layer "F.Cu") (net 1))
 (segment (start 136.32 87.91) (end 136.32 86.8256) (width 0.2) (layer "F.Cu") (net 1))
 (segment (start 149.1234 82.7408) (end 148.395199 83.469001) (width 0.2) (layer "F.Cu") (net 1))
 (segment (start 145.384001 83.469001) (end 146.66 83.469001) (width 0.2) (layer "F.Cu") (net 1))
 (segment (start 136.25 80.3) (end 136.2 80.25) (width 0.2) (layer "F.Cu") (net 1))
 (segment (start 137.6934 86.3222) (end 135.8166 86.3222) (width 0.2) (layer "F.Cu") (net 1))
 (segment (start 139.792 78.053) (end 139.29 78.555) (width 0.2) (layer "F.Cu") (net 1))
 (segment (start 135.8166 86.3222) (end 135.7884 86.294) (width 0.2) (layer "F.Cu") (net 1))
 (via (at 145.97 85.27) (size 0.6) (drill 0.3) (layers "F.Cu" "B.Cu") (free yes) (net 1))
 (via (at 136.32 87.91) (size 0.6) (drill 0.3) (layers "F.Cu" "B.Cu") (free yes) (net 1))
 (via (at 140.345 81.255) (size 0.6) (drill 0.3) (layers "F.Cu" "B.Cu") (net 1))
 (via (at 138.09 79.34) (size 0.6) (drill 0.3) (layers "F.Cu" "B.Cu") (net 1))
 (via (at 136.2 80.25) (size 0.6) (drill 0.3) (layers "F.Cu" "B.Cu") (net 1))
 (segment (start 138.09 79.34) (end 135.99 79.34) (width 0.2) (layer "B.Cu") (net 1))
 (segment (start 135.99 80.04) (end 136.2 80.25) (width 0.2) (layer "B.Cu") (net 1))
 (segment (start 135.99 79.34) (end 135.99 80.04) (width 0.2) (layer "B.Cu") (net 1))
 (segment (start 139.290057 77.29) (end 142.54 77.29) (width 0.2) (layer "F.Cu") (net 5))
 (segment (start 143.4394 78.1894) (end 143.4394 79.5044) (width 0.2) (layer "F.Cu") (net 5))
 (segment (start 142.54 77.29) (end 143.4394 78.1894) (width 0.2) (layer "F.Cu") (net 5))
 (segment (start 137.841057 79.941) (end 137.489 79.588943) (width 0.2) (layer "F.Cu") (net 5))
 (segment (start 143.0644 79.8794) (end 143.0644 81.3934) (width 0.2) (layer "F.Cu") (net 5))
 (segment (start 137.489 79.588943) (end 137.489 79.091057) (width 0.2) (layer "F.Cu") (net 5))
 (segment (start 142.705 82.34) (end 142.423601 82.621399) (width 0.2) (layer "F.Cu") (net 5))
 (segment (start 141.836401 82.621399) (end 141.133401 82.621399) (width 0.2) (layer "F.Cu") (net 5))
 (segment (start 143.4394 79.5044) (end 143.0644 79.8794) (width 0.2) (layer "F.Cu") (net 5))
 (segment (start 137.489 79.091057) (end 139.290057 77.29) (width 0.2) (layer "F.Cu") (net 5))
 (segment (start 139.333399 80.935456) (end 138.338943 79.941) (width 0.2) (layer "F.Cu") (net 5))
 (segment (start 138.338943 79.941) (end 137.841057 79.941) (width 0.2) (layer "F.Cu") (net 5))
 (segment (start 143.0644 81.3934) (end 141.836401 82.621399) (width 0.2) (layer "F.Cu") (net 5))
 (segment (start 142.423601 82.621399) (end 141.133401 82.621399) (width 0.2) (layer "F.Cu") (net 5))
 (segment (start 139.333399 82.133399) (end 139.333399 80.935456) (width 0.2) (layer "F.Cu") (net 5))
 (segment (start 148.445999 80.513399) (end 146.66 80.513399) (width 0.2) (layer "F.Cu") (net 2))
 (segment (start 149.1234 81.1908) (end 148.445999 80.513399) (width 0.2) (layer "F.Cu") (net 2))
 (segment (start 149.1234 81.1908) (end 149.6692 81.1908) (width 0.2) (layer "F.Cu") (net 2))
 (segment (start 147.1782 90.515) (end 153.0858 84.6074) (width 0.2) (layer "F.Cu") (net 2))
 (segment (start 144.2088 78.7146) (end 144.2088 80.257) (width 0.2) (layer "F.Cu") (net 2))
 (segment (start 149.6692 81.1908) (end 153.0858 84.6074) (width 0.2) (layer "F.Cu") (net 2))
 (segment (start 146.121599 80.6704) (end 146.2786 80.513399) (width 0.2) (layer "F.Cu") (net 2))
 (segment (start 146.502999 80.6704) (end 146.66 80.513399) (width 0.2) (layer "F.Cu") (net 2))
 (segment (start 143.7954 80.6704) (end 146.502999 80.6704) (width 0.2) (layer "F.Cu") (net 2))
 (segment (start 147.1782 92.6846) (end 147.1782 90.515) (width 0.2) (layer "F.Cu") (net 2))
 (segment (start 144.2088 80.257) (end 143.7954 80.6704) (width 0.2) (layer "F.Cu") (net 2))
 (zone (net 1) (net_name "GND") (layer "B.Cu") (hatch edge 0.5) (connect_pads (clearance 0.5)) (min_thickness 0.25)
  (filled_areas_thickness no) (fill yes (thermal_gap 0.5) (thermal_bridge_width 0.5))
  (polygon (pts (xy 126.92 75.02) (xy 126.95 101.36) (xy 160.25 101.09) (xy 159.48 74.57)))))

